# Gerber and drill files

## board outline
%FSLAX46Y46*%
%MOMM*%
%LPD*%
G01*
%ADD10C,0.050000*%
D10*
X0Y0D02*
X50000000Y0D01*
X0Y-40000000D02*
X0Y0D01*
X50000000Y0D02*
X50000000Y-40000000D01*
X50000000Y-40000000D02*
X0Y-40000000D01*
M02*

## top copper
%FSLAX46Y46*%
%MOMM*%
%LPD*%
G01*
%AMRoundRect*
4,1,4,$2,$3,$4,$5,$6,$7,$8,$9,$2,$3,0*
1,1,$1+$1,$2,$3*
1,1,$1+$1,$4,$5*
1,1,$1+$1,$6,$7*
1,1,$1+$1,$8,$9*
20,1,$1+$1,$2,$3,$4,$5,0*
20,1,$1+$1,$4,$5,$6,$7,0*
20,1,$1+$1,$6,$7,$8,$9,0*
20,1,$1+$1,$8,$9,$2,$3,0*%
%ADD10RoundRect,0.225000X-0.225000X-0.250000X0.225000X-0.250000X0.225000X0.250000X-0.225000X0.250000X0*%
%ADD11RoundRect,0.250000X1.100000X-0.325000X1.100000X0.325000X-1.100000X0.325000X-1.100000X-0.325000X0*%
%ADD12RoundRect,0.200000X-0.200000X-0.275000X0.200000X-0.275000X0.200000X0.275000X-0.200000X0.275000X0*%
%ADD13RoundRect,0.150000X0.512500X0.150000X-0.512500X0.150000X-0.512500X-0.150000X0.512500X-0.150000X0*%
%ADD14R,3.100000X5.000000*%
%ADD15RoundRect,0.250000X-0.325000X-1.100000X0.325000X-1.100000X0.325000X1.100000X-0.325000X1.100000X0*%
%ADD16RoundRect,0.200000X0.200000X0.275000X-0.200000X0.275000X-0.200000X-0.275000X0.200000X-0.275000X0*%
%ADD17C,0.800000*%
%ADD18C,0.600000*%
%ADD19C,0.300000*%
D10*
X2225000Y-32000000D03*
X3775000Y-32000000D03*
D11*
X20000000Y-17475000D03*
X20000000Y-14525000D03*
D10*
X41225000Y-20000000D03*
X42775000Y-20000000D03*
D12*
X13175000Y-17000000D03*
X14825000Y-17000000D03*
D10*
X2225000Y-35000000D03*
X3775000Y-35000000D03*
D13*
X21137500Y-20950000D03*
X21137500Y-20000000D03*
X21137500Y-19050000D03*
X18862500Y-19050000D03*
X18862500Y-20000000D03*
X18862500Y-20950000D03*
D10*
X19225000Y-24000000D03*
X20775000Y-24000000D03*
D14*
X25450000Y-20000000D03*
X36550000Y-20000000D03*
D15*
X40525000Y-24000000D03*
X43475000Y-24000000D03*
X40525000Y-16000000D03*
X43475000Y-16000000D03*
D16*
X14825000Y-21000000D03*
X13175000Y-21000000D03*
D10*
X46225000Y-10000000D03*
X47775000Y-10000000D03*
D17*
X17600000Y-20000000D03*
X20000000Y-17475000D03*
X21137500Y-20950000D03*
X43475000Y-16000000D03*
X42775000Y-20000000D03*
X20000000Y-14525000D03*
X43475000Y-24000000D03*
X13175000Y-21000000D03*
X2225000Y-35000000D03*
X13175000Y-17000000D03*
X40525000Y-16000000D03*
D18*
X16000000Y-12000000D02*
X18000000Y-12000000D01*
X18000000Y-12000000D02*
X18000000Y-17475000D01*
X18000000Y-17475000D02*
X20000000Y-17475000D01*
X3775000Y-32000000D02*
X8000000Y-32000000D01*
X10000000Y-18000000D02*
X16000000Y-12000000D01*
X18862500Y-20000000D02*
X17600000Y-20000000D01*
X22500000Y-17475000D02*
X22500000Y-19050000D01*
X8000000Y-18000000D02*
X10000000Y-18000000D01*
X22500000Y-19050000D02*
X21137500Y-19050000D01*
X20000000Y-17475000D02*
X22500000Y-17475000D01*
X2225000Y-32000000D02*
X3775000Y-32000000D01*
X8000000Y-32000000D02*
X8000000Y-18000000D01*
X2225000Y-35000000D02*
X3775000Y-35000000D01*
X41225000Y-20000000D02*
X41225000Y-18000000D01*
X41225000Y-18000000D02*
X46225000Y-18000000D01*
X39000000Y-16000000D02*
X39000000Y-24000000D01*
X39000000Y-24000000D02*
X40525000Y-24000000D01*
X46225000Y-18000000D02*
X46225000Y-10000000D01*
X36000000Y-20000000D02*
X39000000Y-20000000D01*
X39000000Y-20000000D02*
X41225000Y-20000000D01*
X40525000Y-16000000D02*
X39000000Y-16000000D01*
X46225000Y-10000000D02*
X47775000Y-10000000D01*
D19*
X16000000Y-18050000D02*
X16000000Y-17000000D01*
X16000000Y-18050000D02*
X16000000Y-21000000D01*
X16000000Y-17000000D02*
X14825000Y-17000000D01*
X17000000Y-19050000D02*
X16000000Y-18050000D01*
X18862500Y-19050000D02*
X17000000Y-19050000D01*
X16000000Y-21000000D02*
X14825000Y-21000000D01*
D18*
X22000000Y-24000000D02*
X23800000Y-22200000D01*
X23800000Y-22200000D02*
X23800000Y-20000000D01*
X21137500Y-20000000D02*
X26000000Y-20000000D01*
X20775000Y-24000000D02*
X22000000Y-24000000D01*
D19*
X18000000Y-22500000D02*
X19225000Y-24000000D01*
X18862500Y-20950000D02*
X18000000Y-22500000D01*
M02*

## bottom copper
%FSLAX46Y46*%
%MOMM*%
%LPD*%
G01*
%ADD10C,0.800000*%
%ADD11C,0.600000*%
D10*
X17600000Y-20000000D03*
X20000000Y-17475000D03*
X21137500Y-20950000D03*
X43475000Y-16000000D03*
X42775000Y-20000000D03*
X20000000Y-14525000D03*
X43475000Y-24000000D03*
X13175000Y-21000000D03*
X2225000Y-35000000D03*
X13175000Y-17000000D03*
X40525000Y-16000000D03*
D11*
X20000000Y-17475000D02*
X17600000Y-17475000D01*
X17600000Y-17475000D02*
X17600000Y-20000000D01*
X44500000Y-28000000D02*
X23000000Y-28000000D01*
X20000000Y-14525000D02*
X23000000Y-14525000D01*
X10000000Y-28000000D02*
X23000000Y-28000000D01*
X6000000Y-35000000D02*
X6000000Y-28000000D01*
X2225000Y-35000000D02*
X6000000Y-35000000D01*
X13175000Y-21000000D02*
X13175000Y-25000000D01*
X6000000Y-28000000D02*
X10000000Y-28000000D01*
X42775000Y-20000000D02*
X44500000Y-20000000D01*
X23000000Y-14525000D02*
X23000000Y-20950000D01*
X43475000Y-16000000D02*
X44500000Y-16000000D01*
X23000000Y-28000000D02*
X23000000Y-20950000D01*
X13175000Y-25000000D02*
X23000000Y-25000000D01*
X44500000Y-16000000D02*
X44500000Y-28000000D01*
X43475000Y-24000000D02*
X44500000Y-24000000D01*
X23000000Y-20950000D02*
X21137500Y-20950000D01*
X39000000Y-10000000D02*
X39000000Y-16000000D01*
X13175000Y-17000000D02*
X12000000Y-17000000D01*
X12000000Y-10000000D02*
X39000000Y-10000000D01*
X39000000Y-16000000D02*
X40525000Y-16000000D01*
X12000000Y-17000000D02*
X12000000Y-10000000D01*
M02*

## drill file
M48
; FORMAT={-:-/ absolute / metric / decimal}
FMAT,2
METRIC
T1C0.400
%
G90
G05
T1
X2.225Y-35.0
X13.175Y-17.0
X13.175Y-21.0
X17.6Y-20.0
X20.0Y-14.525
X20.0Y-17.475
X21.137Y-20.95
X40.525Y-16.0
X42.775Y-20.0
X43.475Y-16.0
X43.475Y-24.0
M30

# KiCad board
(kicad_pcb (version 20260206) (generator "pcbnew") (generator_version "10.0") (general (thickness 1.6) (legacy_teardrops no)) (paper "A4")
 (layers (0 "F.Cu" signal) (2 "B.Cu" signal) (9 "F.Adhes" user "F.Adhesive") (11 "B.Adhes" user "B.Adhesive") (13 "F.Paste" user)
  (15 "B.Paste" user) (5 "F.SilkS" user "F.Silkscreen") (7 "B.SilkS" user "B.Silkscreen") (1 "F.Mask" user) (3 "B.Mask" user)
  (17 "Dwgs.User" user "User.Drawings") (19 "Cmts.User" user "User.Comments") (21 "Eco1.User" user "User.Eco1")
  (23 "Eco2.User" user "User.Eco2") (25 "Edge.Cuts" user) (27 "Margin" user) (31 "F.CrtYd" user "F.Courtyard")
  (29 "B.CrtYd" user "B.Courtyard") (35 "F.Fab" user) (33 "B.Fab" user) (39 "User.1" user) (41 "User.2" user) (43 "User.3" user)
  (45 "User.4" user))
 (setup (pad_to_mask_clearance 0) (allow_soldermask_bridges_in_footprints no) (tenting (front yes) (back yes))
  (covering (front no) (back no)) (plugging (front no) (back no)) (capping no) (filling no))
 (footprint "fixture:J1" (layer "F.Cu") (at 3 32)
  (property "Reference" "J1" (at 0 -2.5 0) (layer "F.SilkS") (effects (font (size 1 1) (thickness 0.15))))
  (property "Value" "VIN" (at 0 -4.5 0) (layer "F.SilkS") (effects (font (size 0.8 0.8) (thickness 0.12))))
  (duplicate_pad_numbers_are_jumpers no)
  (pad "1" smd roundrect (at -0.775 0) (size 0.9 0.95) (layers "F.Cu" "F.Mask" "F.Paste") (roundrect_rratio 0.25) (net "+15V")
   (thermal_bridge_angle 45))
  (pad "2" smd roundrect (at 0.775 0) (size 0.9 0.95) (layers "F.Cu" "F.Mask" "F.Paste") (roundrect_rratio 0.25) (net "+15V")
   (thermal_bridge_angle 45)))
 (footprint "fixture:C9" (layer "F.Cu") (at 20 16 90)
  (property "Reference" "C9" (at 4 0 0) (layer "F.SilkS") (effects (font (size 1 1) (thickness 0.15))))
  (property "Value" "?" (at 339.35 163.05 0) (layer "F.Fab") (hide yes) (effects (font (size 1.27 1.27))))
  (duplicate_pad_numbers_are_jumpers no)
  (pad "1" smd roundrect (at -1.475 0 90) (size 1.15 2.7) (layers "F.Cu" "F.Mask" "F.Paste") (roundrect_rratio 0.217391) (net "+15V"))
  (pad "2" smd roundrect (at 1.475 0 90) (size 1.15 2.7) (layers "F.Cu" "F.Mask" "F.Paste") (roundrect_rratio 0.217391) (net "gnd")))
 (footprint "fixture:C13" (layer "F.Cu") (at 42 20)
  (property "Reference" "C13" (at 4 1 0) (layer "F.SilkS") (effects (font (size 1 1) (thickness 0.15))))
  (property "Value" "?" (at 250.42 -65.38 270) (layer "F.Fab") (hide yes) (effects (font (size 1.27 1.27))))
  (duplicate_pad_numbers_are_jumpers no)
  (pad "1" smd roundrect (at -0.775 0) (size 0.9 0.95) (layers "F.Cu" "F.Mask" "F.Paste") (roundrect_rratio 0.25) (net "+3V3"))
  (pad "2" smd roundrect (at 0.775 0) (size 0.9 0.95) (layers "F.Cu" "F.Mask" "F.Paste") (roundrect_rratio 0.25) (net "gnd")))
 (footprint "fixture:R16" (layer "F.Cu") (at 14 17)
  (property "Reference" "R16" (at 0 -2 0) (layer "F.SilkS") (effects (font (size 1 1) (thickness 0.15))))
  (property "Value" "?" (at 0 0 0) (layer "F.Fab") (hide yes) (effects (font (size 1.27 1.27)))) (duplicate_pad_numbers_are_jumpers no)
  (pad "1" smd roundrect (at -0.825 0) (size 0.8 0.95) (layers "F.Cu" "F.Mask" "F.Paste") (roundrect_rratio 0.25) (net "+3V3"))
  (pad "2" smd roundrect (at 0.825 0) (size 0.8 0.95) (layers "F.Cu" "F.Mask" "F.Paste") (roundrect_rratio 0.25) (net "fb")))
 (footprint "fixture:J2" (layer "F.Cu") (at 3 35)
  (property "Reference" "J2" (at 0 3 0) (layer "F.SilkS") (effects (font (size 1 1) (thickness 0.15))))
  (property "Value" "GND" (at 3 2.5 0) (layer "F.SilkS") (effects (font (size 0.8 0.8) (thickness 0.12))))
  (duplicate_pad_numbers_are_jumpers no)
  (pad "1" smd roundrect (at -0.775 0) (size 0.9 0.95) (layers "F.Cu" "F.Mask" "F.Paste") (roundrect_rratio 0.25) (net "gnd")
   (thermal_bridge_angle 45))
  (pad "2" smd roundrect (at 0.775 0) (size 0.9 0.95) (layers "F.Cu" "F.Mask" "F.Paste") (roundrect_rratio 0.25) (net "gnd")
   (thermal_bridge_angle 45)))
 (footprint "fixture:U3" (layer "F.Cu") (at 20 20 180)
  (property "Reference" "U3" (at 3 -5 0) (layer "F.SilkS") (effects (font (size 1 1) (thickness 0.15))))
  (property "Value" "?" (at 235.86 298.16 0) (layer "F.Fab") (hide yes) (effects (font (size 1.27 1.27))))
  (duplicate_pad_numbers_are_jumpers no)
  (pad "1" smd roundrect (at -1.1375 -0.95 180) (size 1.325 0.6) (layers "F.Cu" "F.Mask" "F.Paste") (roundrect_rratio 0.25) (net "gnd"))
  (pad "2" smd roundrect (at -1.1375 0 180) (size 1.325 0.6) (layers "F.Cu" "F.Mask" "F.Paste") (roundrect_rratio 0.25) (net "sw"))
  (pad "3" smd roundrect (at -1.1375 0.95 180) (size 1.325 0.6) (layers "F.Cu" "F.Mask" "F.Paste") (roundrect_rratio 0.25) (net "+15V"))
  (pad "4" smd roundrect (at 1.1375 0.95 180) (size 1.325 0.6) (layers "F.Cu" "F.Mask" "F.Paste") (roundrect_rratio 0.25) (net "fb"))
  (pad "5" smd roundrect (at 1.1375 0 180) (size 1.325 0.6) (layers "F.Cu" "F.Mask" "F.Paste") (roundrect_rratio 0.25) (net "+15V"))
  (pad "6" smd roundrect (at 1.1375 -0.95 180) (size 1.325 0.6) (layers "F.Cu" "F.Mask" "F.Paste") (roundrect_rratio 0.25) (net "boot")))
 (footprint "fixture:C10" (layer "F.Cu") (at 20 24)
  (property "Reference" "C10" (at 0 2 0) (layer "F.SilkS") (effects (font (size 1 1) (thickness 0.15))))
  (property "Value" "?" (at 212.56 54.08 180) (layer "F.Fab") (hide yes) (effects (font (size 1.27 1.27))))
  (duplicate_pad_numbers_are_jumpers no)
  (pad "1" smd roundrect (at -0.775 0) (size 0.9 0.95) (layers "F.Cu" "F.Mask" "F.Paste") (roundrect_rratio 0.25) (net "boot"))
  (pad "2" smd roundrect (at 0.775 0) (size 0.9 0.95) (layers "F.Cu" "F.Mask" "F.Paste") (roundrect_rratio 0.25) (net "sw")))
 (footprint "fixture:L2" (layer "F.Cu") (at 31 20)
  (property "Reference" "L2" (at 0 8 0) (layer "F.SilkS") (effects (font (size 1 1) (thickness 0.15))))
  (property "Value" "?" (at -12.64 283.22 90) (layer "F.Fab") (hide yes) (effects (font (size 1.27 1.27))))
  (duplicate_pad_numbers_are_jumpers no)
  (pad "1" smd rect (at -5.55 0) (size 3.1 5) (layers "F.Cu" "F.Mask" "F.Paste") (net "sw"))
  (pad "2" smd rect (at 5.55 0) (size 3.1 5) (layers "F.Cu" "F.Mask" "F.Paste") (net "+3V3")))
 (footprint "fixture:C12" (layer "F.Cu") (at 42 24)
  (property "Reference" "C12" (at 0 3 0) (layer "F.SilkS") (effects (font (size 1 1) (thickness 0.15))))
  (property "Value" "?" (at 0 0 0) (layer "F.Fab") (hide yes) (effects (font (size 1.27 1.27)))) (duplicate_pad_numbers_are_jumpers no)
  (pad "1" smd roundrect (at -1.475 0) (size 1.15 2.7) (layers "F.Cu" "F.Mask" "F.Paste") (roundrect_rratio 0.217391) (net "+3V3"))
  (pad "2" smd roundrect (at 1.475 0) (size 1.15 2.7) (layers "F.Cu" "F.Mask" "F.Paste") (roundrect_rratio 0.217391) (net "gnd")))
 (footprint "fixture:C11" (layer "F.Cu") (at 42 16)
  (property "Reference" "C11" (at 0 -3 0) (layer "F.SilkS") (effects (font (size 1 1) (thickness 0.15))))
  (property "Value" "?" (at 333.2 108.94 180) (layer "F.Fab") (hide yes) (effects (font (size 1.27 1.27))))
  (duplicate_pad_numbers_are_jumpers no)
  (pad "1" smd roundrect (at -1.475 0) (size 1.15 2.7) (layers "F.Cu" "F.Mask" "F.Paste") (roundrect_rratio 0.217391) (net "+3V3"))
  (pad "2" smd roundrect (at 1.475 0) (size 1.15 2.7) (layers "F.Cu" "F.Mask" "F.Paste") (roundrect_rratio 0.217391) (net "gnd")))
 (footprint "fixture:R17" (layer "F.Cu") (at 14 21 180)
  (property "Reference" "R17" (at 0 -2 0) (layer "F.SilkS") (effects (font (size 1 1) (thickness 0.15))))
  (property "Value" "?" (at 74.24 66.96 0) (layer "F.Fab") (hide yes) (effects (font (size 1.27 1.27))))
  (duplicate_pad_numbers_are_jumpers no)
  (pad "1" smd roundrect (at -0.825 0 180) (size 0.8 0.95) (layers "F.Cu" "F.Mask" "F.Paste") (roundrect_rratio 0.25) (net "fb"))
  (pad "2" smd roundrect (at 0.825 0 180) (size 0.8 0.95) (layers "F.Cu" "F.Mask" "F.Paste") (roundrect_rratio 0.25) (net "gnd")))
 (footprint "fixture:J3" (layer "F.Cu") (at 47 10)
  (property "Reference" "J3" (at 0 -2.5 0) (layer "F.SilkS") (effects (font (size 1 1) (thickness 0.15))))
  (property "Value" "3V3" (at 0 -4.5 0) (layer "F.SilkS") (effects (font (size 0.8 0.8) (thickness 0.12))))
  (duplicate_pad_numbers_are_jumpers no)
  (pad "1" smd roundrect (at -0.775 0) (size 0.9 0.95) (layers "F.Cu" "F.Mask" "F.Paste") (roundrect_rratio 0.25) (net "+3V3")
   (thermal_bridge_angle 45))
  (pad "2" smd roundrect (at 0.775 0) (size 0.9 0.95) (layers "F.Cu" "F.Mask" "F.Paste") (roundrect_rratio 0.25) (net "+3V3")
   (thermal_bridge_angle 45)))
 (gr_line (start 0 0) (end 50 0) (stroke (width 0.05) (type default)) (layer "Edge.Cuts"))
 (gr_line (start 0 40) (end 0 0) (stroke (width 0.05) (type default)) (layer "Edge.Cuts"))
 (gr_line (start 50 0) (end 50 40) (stroke (width 0.05) (type default)) (layer "Edge.Cuts"))
 (gr_line (start 50 40) (end 0 40) (stroke (width 0.05) (type default)) (layer "Edge.Cuts"))
 (segment (start 16 12) (end 18 12) (width 0.6) (layer "F.Cu") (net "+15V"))
 (segment (start 18 12) (end 18 17.475) (width 0.6) (layer "F.Cu") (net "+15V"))
 (segment (start 18 17.475) (end 20 17.475) (width 0.6) (layer "F.Cu") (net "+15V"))
 (segment (start 3.775 32) (end 8 32) (width 0.6) (layer "F.Cu") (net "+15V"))
 (segment (start 10 18) (end 16 12) (width 0.6) (layer "F.Cu") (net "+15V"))
 (segment (start 18.8625 20) (end 17.6 20) (width 0.6) (layer "F.Cu") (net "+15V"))
 (segment (start 22.5 17.475) (end 22.5 19.05) (width 0.6) (layer "F.Cu") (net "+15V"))
 (segment (start 8 18) (end 10 18) (width 0.6) (layer "F.Cu") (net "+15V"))
 (segment (start 22.5 19.05) (end 21.1375 19.05) (width 0.6) (layer "F.Cu") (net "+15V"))
 (segment (start 20 17.475) (end 22.5 17.475) (width 0.6) (layer "F.Cu") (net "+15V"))
 (segment (start 2.225 32) (end 3.775 32) (width 0.6) (layer "F.Cu") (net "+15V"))
 (segment (start 8 32) (end 8 18) (width 0.6) (layer "F.Cu") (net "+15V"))
 (via (at 17.6 20) (size 0.8) (drill 0.4) (layers "F.Cu" "B.Cu") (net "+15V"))
 (via (at 20 17.475) (size 0.8) (drill 0.4) (layers "F.Cu" "B.Cu") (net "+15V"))
 (segment (start 20 17.475) (end 17.6 17.475) (width 0.6) (layer "B.Cu") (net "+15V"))
 (segment (start 17.6 17.475) (end 17.6 20) (width 0.6) (layer "B.Cu") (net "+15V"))
 (segment (start 2.225 35) (end 3.775 35) (width 0.6) (layer "F.Cu") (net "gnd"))
 (via (at 21.1375 20.95) (size 0.8) (drill 0.4) (layers "F.Cu" "B.Cu") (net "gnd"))
 (via (at 43.475 16) (size 0.8) (drill 0.4) (layers "F.Cu" "B.Cu") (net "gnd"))
 (via (at 42.775 20) (size 0.8) (drill 0.4) (layers "F.Cu" "B.Cu") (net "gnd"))
 (via (at 20 14.525) (size 0.8) (drill 0.4) (layers "F.Cu" "B.Cu") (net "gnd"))
 (via (at 43.475 24) (size 0.8) (drill 0.4) (layers "F.Cu" "B.Cu") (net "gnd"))
 (via (at 13.175 21) (size 0.8) (drill 0.4) (layers "F.Cu" "B.Cu") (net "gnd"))
 (via (at 2.225 35) (size 0.8) (drill 0.4) (layers "F.Cu" "B.Cu") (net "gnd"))
 (segment (start 44.5 28) (end 23 28) (width 0.6) (layer "B.Cu") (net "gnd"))
 (segment (start 20 14.525) (end 23 14.525) (width 0.6) (layer "B.Cu") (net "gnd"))
 (segment (start 10 28) (end 23 28) (width 0.6) (layer "B.Cu") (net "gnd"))
 (segment (start 6 35) (end 6 28) (width 0.6) (layer "B.Cu") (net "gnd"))
 (segment (start 2.225 35) (end 6 35) (width 0.6) (layer "B.Cu") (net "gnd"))
 (segment (start 13.175 21) (end 13.175 25) (width 0.6) (layer "B.Cu") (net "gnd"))
 (segment (start 6 28) (end 10 28) (width 0.6) (layer "B.Cu") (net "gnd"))
 (segment (start 42.775 20) (end 44.5 20) (width 0.6) (layer "B.Cu") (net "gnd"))
 (segment (start 23 14.525) (end 23 20.95) (width 0.6) (layer "B.Cu") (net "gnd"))
 (segment (start 43.475 16) (end 44.5 16) (width 0.6) (layer "B.Cu") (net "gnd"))
 (segment (start 23 28) (end 23 20.95) (width 0.6) (layer "B.Cu") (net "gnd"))
 (segment (start 13.175 25) (end 23 25) (width 0.6) (layer "B.Cu") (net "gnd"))
 (segment (start 44.5 16) (end 44.5 28) (width 0.6) (layer "B.Cu") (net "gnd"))
 (segment (start 43.475 24) (end 44.5 24) (width 0.6) (layer "B.Cu") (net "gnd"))
 (segment (start 23 20.95) (end 21.1375 20.95) (width 0.6) (layer "B.Cu") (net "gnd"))
 (segment (start 41.225 20) (end 41.225 18) (width 0.6) (layer "F.Cu") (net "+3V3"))
 (segment (start 41.225 18) (end 46.225 18) (width 0.6) (layer "F.Cu") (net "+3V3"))
 (segment (start 39 16) (end 39 24) (width 0.6) (layer "F.Cu") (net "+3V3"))
 (segment (start 39 24) (end 40.525 24) (width 0.6) (layer "F.Cu") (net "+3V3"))
 (segment (start 46.225 18) (end 46.225 10) (width 0.6) (layer "F.Cu") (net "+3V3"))
 (segment (start 36 20) (end 39 20) (width 0.6) (layer "F.Cu") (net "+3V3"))
 (segment (start 39 20) (end 41.225 20) (width 0.6) (layer "F.Cu") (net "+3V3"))
 (segment (start 40.525 16) (end 39 16) (width 0.6) (layer "F.Cu") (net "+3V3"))
 (segment (start 46.225 10) (end 47.775 10) (width 0.6) (layer "F.Cu") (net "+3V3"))
 (via (at 13.175 17) (size 0.8) (drill 0.4) (layers "F.Cu" "B.Cu") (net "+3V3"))
 (via (at 40.525 16) (size 0.8) (drill 0.4) (layers "F.Cu" "B.Cu") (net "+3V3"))
 (segment (start 39 10) (end 39 16) (width 0.6) (layer "B.Cu") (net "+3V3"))
 (segment (start 13.175 17) (end 12 17) (width 0.6) (layer "B.Cu") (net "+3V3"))
 (segment (start 12 10) (end 39 10) (width 0.6) (layer "B.Cu") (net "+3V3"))
 (segment (start 39 16) (end 40.525 16) (width 0.6) (layer "B.Cu") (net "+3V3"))
 (segment (start 12 17) (end 12 10) (width 0.6) (layer "B.Cu") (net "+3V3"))
 (segment (start 16 18.05) (end 16 17) (width 0.3) (layer "F.Cu") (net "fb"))
 (segment (start 16 18.05) (end 16 21) (width 0.3) (layer "F.Cu") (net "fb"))
 (segment (start 16 17) (end 14.825 17) (width 0.3) (layer "F.Cu") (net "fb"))
 (segment (start 17 19.05) (end 16 18.05) (width 0.3) (layer "F.Cu") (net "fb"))
 (segment (start 18.8625 19.05) (end 17 19.05) (width 0.3) (layer "F.Cu") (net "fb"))
 (segment (start 16 21) (end 14.825 21) (width 0.3) (layer "F.Cu") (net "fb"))
 (segment (start 22 24) (end 23.8 22.2) (width 0.6) (layer "F.Cu") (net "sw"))
 (segment (start 23.8 22.2) (end 23.8 20) (width 0.6) (layer "F.Cu") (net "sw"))
 (segment (start 21.1375 20) (end 26 20) (width 0.6) (layer "F.Cu") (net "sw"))
 (segment (start 20.775 24) (end 22 24) (width 0.6) (layer "F.Cu") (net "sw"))
 (segment (start 18 22.5) (end 19.225 24) (width 0.3) (layer "F.Cu") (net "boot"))
 (segment (start 18.8625 20.95) (end 18 22.5) (width 0.3) (layer "F.Cu") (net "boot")))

